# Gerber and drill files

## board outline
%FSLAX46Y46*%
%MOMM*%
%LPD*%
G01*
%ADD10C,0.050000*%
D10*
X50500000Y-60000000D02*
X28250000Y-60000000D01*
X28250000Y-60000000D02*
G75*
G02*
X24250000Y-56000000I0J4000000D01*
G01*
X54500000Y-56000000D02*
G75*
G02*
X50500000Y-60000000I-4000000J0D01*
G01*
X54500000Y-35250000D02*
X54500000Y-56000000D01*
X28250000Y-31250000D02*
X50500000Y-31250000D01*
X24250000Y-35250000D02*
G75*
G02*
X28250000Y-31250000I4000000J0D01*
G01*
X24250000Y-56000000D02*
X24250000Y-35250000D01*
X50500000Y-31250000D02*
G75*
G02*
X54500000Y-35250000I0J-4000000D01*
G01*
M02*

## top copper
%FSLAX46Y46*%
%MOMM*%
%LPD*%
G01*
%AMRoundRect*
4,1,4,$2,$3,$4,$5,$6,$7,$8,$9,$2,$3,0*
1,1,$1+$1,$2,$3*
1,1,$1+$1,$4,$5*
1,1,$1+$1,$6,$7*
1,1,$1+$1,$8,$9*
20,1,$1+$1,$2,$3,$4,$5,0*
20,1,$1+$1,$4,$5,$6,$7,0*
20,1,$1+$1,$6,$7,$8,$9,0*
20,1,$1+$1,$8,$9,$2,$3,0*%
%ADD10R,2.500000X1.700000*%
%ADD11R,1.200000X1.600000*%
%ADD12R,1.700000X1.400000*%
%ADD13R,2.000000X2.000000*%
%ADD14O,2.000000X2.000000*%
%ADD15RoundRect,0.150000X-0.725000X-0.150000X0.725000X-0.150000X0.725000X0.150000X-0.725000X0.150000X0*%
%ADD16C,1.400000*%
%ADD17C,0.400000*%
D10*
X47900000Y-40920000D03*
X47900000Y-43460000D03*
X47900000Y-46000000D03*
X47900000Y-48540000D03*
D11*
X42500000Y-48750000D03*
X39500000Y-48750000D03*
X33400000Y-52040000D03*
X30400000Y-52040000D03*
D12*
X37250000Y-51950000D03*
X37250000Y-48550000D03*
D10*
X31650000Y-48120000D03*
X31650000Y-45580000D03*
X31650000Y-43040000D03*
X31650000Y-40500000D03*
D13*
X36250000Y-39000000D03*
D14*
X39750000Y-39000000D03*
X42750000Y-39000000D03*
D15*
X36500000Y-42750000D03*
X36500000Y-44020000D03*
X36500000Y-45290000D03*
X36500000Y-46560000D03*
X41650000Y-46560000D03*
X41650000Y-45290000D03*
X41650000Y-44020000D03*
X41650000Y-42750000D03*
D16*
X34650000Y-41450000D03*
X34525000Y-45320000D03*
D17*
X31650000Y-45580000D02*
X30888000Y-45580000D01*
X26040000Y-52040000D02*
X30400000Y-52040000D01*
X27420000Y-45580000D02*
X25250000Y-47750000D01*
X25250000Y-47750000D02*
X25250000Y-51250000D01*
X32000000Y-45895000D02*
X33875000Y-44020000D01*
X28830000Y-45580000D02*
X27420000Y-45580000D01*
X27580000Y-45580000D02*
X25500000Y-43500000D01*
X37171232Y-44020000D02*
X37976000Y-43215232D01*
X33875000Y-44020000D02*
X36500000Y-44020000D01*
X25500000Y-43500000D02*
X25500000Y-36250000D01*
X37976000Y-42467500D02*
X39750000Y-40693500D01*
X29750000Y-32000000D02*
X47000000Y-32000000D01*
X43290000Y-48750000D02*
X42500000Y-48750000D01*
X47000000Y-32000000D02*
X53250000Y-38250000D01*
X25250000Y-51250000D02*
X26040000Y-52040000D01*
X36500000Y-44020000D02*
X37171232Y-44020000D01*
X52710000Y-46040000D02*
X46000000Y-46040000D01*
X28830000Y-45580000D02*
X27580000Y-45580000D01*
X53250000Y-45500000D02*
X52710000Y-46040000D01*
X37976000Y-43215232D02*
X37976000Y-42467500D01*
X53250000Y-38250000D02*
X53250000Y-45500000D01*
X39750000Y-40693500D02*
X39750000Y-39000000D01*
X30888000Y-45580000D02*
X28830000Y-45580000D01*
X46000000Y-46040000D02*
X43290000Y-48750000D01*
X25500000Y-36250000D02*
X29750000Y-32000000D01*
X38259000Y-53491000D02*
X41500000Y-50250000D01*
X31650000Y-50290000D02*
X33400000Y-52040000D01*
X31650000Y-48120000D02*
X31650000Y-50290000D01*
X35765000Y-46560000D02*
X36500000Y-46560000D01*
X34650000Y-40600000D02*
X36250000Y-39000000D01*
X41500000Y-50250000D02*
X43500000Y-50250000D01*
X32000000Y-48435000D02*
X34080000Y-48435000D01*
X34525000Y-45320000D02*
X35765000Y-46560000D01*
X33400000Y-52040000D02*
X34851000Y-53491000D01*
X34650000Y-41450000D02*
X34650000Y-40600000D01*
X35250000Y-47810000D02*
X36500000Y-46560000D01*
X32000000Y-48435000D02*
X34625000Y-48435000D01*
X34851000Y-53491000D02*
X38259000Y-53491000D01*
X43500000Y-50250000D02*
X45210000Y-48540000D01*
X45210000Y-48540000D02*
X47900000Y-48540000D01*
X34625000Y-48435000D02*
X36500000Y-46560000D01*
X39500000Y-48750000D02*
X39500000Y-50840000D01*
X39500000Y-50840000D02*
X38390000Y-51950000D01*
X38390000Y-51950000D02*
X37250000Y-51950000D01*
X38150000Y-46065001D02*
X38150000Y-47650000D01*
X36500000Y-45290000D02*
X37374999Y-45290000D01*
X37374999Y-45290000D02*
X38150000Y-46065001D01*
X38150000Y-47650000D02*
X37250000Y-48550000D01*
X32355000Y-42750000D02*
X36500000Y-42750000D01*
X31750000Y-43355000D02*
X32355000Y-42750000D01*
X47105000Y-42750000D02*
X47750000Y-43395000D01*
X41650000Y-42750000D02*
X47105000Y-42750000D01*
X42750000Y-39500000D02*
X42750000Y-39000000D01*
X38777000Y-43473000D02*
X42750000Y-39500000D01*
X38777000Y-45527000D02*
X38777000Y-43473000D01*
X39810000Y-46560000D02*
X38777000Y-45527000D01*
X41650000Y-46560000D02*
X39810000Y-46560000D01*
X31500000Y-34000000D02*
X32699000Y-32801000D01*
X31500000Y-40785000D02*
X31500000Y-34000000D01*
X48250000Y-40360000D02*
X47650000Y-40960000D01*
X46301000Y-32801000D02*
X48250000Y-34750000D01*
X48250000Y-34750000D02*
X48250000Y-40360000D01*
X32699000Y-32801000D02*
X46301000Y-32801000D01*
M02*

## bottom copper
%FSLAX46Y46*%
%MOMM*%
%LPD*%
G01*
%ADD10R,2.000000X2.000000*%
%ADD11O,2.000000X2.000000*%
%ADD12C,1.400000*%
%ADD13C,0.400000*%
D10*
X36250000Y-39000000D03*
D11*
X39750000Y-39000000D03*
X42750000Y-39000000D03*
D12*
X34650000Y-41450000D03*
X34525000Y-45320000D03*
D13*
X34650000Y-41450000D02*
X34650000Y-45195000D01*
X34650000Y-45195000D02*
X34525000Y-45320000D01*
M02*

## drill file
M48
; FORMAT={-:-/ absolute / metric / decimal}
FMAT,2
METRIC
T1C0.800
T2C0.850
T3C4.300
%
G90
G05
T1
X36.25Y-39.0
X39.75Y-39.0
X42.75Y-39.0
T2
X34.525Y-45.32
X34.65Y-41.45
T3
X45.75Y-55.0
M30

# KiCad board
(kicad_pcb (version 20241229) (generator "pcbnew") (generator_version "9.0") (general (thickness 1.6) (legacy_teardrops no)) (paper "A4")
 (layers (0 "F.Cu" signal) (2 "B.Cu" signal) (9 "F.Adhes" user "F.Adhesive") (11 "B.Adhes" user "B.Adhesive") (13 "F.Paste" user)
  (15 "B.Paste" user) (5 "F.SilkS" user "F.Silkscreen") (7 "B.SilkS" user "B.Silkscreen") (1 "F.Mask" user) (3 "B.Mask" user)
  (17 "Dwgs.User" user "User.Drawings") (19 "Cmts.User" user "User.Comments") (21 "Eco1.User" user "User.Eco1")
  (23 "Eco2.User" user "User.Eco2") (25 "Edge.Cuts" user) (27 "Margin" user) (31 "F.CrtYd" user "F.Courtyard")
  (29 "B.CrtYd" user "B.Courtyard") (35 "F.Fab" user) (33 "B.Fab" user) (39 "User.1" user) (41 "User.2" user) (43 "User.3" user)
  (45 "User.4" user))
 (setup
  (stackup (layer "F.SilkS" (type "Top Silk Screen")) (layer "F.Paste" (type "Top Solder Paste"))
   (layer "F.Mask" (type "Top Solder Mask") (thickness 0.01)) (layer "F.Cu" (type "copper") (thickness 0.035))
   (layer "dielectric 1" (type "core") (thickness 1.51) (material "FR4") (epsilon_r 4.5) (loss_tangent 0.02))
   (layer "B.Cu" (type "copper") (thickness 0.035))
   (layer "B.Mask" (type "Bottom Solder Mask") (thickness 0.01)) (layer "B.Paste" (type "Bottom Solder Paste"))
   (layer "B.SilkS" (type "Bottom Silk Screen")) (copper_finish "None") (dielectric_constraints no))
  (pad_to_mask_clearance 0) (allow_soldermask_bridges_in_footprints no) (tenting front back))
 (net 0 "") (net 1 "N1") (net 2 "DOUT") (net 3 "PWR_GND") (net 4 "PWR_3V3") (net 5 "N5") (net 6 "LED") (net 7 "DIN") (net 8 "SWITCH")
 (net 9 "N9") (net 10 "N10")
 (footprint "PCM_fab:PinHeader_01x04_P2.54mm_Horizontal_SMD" (layer "F.Cu") (at 47.9 40.92)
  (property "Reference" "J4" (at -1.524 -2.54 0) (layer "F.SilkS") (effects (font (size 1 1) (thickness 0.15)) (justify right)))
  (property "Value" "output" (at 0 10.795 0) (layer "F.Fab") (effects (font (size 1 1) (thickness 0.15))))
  (pad "1" smd rect (at 0 0) (size 2.5 1.7) (layers "F.Cu" "F.Mask" "F.Paste") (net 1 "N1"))
  (pad "2" smd rect (at 0 2.54) (size 2.5 1.7) (layers "F.Cu" "F.Mask" "F.Paste") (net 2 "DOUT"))
  (pad "3" smd rect (at 0 5.08) (size 2.5 1.7) (layers "F.Cu" "F.Mask" "F.Paste") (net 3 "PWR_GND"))
  (pad "4" smd rect (at 0 7.62) (size 2.5 1.7) (layers "F.Cu" "F.Mask" "F.Paste") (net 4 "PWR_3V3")))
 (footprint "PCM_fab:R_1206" (layer "F.Cu") (at 41 48.75 180)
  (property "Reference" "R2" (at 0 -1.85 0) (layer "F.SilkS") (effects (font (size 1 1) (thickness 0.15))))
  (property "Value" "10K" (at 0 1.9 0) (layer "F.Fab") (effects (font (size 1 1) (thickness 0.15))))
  (pad "1" smd rect (at -1.5 0 180) (size 1.2 1.6) (layers "F.Cu" "F.Mask" "F.Paste") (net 3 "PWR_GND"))
  (pad "2" smd rect (at 1.5 0 180) (size 1.2 1.6) (layers "F.Cu" "F.Mask" "F.Paste") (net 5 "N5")))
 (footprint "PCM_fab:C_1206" (layer "F.Cu") (at 31.9 52.04 180)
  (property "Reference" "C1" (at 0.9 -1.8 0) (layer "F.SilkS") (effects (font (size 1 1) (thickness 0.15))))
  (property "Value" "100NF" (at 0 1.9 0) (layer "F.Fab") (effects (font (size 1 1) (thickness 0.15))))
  (pad "1" smd rect (at -1.5 0 180) (size 1.2 1.6) (layers "F.Cu" "F.Mask" "F.Paste") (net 4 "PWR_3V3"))
  (pad "2" smd rect (at 1.5 0 180) (size 1.2 1.6) (layers "F.Cu" "F.Mask" "F.Paste") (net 3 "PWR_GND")))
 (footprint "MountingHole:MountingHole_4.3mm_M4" (layer "F.Cu") (at 45.75 55)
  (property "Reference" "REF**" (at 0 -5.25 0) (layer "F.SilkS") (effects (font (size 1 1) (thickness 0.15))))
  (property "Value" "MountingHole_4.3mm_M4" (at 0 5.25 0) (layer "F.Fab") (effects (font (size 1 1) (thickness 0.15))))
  (pad "" np_thru_hole circle (at 0 0) (size 4.3 4.3) (drill 4.3) (layers "*.Cu" "*.Mask")))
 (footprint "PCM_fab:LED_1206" (layer "F.Cu") (at 37.25 50.25 90)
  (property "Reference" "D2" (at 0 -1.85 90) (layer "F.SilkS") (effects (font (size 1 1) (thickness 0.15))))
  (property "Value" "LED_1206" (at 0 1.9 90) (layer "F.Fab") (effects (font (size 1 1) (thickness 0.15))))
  (pad "1" smd rect (at -1.7 0 90) (size 1.4 1.7) (layers "F.Cu" "F.Mask" "F.Paste") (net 5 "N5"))
  (pad "2" smd rect (at 1.7 0 90) (size 1.4 1.7) (layers "F.Cu" "F.Mask" "F.Paste") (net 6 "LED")))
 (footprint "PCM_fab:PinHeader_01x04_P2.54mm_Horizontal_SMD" (layer "F.Cu") (at 31.65 48.12 180)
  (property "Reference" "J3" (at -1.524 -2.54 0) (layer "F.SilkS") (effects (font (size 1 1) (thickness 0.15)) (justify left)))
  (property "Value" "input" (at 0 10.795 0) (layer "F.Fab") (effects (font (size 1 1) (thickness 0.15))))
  (pad "1" smd rect (at 0 0 180) (size 2.5 1.7) (layers "F.Cu" "F.Mask" "F.Paste") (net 4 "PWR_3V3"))
  (pad "2" smd rect (at 0 2.54 180) (size 2.5 1.7) (layers "F.Cu" "F.Mask" "F.Paste") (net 3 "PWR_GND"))
  (pad "3" smd rect (at 0 5.08 180) (size 2.5 1.7) (layers "F.Cu" "F.Mask" "F.Paste") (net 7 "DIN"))
  (pad "4" smd rect (at 0 7.62 180) (size 2.5 1.7) (layers "F.Cu" "F.Mask" "F.Paste") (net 1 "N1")))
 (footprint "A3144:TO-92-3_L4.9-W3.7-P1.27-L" (layer "F.Cu") (at 39.75 39)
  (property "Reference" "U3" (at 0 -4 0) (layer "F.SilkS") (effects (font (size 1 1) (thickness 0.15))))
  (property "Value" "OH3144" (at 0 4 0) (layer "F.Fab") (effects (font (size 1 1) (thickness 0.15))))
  (pad "1" thru_hole rect (at -3.5 0) (size 2 2) (drill 0.8) (layers "*.Cu" "*.Mask") (remove_unused_layers no) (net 4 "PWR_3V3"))
  (pad "2" thru_hole oval (at 0 0) (size 2 2) (drill 0.8) (layers "*.Cu" "*.Mask") (remove_unused_layers no) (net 3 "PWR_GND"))
  (pad "3" thru_hole oval (at 3 0) (size 2 2) (drill 0.8) (layers "*.Cu" "*.Mask") (remove_unused_layers no) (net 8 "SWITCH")))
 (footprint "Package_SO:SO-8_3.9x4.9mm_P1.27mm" (layer "F.Cu") (at 39.075 44.655)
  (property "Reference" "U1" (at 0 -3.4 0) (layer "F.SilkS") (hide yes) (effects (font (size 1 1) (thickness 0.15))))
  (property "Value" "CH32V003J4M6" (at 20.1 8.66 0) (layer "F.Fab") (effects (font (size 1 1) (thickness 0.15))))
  (pad "1" smd roundrect (at -2.575 -1.905) (size 1.75 0.6) (layers "F.Cu" "F.Mask" "F.Paste") (roundrect_rratio 0.25) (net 7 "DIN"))
  (pad "2" smd roundrect (at -2.575 -0.635) (size 1.75 0.6) (layers "F.Cu" "F.Mask" "F.Paste") (roundrect_rratio 0.25) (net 3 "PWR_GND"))
  (pad "3" smd roundrect (at -2.575 0.635) (size 1.75 0.6) (layers "F.Cu" "F.Mask" "F.Paste") (roundrect_rratio 0.25) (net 6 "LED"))
  (pad "4" smd roundrect (at -2.575 1.905) (size 1.75 0.6) (layers "F.Cu" "F.Mask" "F.Paste") (roundrect_rratio 0.25) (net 4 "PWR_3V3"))
  (pad "5" smd roundrect (at 2.575 1.905) (size 1.75 0.6) (layers "F.Cu" "F.Mask" "F.Paste") (roundrect_rratio 0.25) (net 8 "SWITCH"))
  (pad "6" smd roundrect (at 2.575 0.635) (size 1.75 0.6) (layers "F.Cu" "F.Mask" "F.Paste") (roundrect_rratio 0.25) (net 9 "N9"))
  (pad "7" smd roundrect (at 2.575 -0.635) (size 1.75 0.6) (layers "F.Cu" "F.Mask" "F.Paste") (roundrect_rratio 0.25) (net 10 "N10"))
  (pad "8" smd roundrect (at 2.575 -1.905) (size 1.75 0.6) (layers "F.Cu" "F.Mask" "F.Paste") (roundrect_rratio 0.25) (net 2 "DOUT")))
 (gr_line (start 50.5 60) (end 28.25 60) (stroke (width 0.05) (type default)) (layer "Edge.Cuts"))
 (gr_arc (start 28.25 60) (mid 25.421573 58.828427) (end 24.25 56) (stroke (width 0.05) (type default)) (layer "Edge.Cuts"))
 (gr_arc (start 54.5 56) (mid 53.328427 58.828427) (end 50.5 60) (stroke (width 0.05) (type default)) (layer "Edge.Cuts"))
 (gr_line (start 54.5 35.25) (end 54.5 56) (stroke (width 0.05) (type default)) (layer "Edge.Cuts"))
 (gr_line (start 28.25 31.25) (end 50.5 31.25) (stroke (width 0.05) (type default)) (layer "Edge.Cuts"))
 (gr_arc (start 24.25 35.25) (mid 25.421573 32.421573) (end 28.25 31.25) (stroke (width 0.05) (type default)) (layer "Edge.Cuts"))
 (gr_line (start 24.25 56) (end 24.25 35.25) (stroke (width 0.05) (type default)) (layer "Edge.Cuts"))
 (gr_arc (start 50.5 31.25) (mid 53.328427 32.421573) (end 54.5 35.25) (stroke (width 0.05) (type default)) (layer "Edge.Cuts"))
 (segment (start 31.65 45.58) (end 30.888 45.58) (width 0.4) (layer "F.Cu") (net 3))
 (segment (start 26.04 52.04) (end 30.4 52.04) (width 0.4) (layer "F.Cu") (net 3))
 (segment (start 27.42 45.58) (end 25.25 47.75) (width 0.4) (layer "F.Cu") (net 3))
 (segment (start 25.25 47.75) (end 25.25 51.25) (width 0.4) (layer "F.Cu") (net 3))
 (segment (start 32 45.895) (end 33.875 44.02) (width 0.4) (layer "F.Cu") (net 3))
 (segment (start 28.83 45.58) (end 27.42 45.58) (width 0.4) (layer "F.Cu") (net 3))
 (segment (start 27.58 45.58) (end 25.5 43.5) (width 0.4) (layer "F.Cu") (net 3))
 (segment (start 37.171232 44.02) (end 37.976 43.215232) (width 0.4) (layer "F.Cu") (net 3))
 (segment (start 33.875 44.02) (end 36.5 44.02) (width 0.4) (layer "F.Cu") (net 3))
 (segment (start 25.5 43.5) (end 25.5 36.25) (width 0.4) (layer "F.Cu") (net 3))
 (segment (start 37.976 42.4675) (end 39.75 40.6935) (width 0.4) (layer "F.Cu") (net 3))
 (segment (start 29.75 32) (end 47 32) (width 0.4) (layer "F.Cu") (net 3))
 (segment (start 43.29 48.75) (end 42.5 48.75) (width 0.4) (layer "F.Cu") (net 3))
 (segment (start 47 32) (end 53.25 38.25) (width 0.4) (layer "F.Cu") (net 3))
 (segment (start 25.25 51.25) (end 26.04 52.04) (width 0.4) (layer "F.Cu") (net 3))
 (segment (start 36.5 44.02) (end 37.171232 44.02) (width 0.4) (layer "F.Cu") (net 3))
 (segment (start 52.71 46.04) (end 46 46.04) (width 0.4) (layer "F.Cu") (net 3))
 (segment (start 28.83 45.58) (end 27.58 45.58) (width 0.4) (layer "F.Cu") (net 3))
 (segment (start 53.25 45.5) (end 52.71 46.04) (width 0.4) (layer "F.Cu") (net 3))
 (segment (start 37.976 43.215232) (end 37.976 42.4675) (width 0.4) (layer "F.Cu") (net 3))
 (segment (start 53.25 38.25) (end 53.25 45.5) (width 0.4) (layer "F.Cu") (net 3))
 (segment (start 39.75 40.6935) (end 39.75 39) (width 0.4) (layer "F.Cu") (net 3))
 (segment (start 30.888 45.58) (end 28.83 45.58) (width 0.4) (layer "F.Cu") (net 3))
 (segment (start 46 46.04) (end 43.29 48.75) (width 0.4) (layer "F.Cu") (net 3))
 (segment (start 25.5 36.25) (end 29.75 32) (width 0.4) (layer "F.Cu") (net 3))
 (segment (start 38.259 53.491) (end 41.5 50.25) (width 0.4) (layer "F.Cu") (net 4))
 (segment (start 31.65 50.29) (end 33.4 52.04) (width 0.4) (layer "F.Cu") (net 4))
 (segment (start 31.65 48.12) (end 31.65 50.29) (width 0.4) (layer "F.Cu") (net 4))
 (segment (start 35.765 46.56) (end 36.5 46.56) (width 0.4) (layer "F.Cu") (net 4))
 (segment (start 34.65 40.6) (end 36.25 39) (width 0.4) (layer "F.Cu") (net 4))
 (segment (start 41.5 50.25) (end 43.5 50.25) (width 0.4) (layer "F.Cu") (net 4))
 (segment (start 32 48.435) (end 34.08 48.435) (width 0.4) (layer "F.Cu") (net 4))
 (segment (start 34.525 45.32) (end 35.765 46.56) (width 0.4) (layer "F.Cu") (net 4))
 (segment (start 33.4 52.04) (end 34.851 53.491) (width 0.4) (layer "F.Cu") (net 4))
 (segment (start 34.65 41.45) (end 34.65 40.6) (width 0.4) (layer "F.Cu") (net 4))
 (segment (start 35.25 47.81) (end 36.5 46.56) (width 0.4) (layer "F.Cu") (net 4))
 (segment (start 32 48.435) (end 34.625 48.435) (width 0.4) (layer "F.Cu") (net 4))
 (segment (start 34.851 53.491) (end 38.259 53.491) (width 0.4) (layer "F.Cu") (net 4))
 (segment (start 43.5 50.25) (end 45.21 48.54) (width 0.4) (layer "F.Cu") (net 4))
 (segment (start 45.21 48.54) (end 47.9 48.54) (width 0.4) (layer "F.Cu") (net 4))
 (segment (start 34.625 48.435) (end 36.5 46.56) (width 0.4) (layer "F.Cu") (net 4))
 (via (at 34.65 41.45) (size 1.4) (drill 0.85) (layers "F.Cu" "B.Cu") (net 4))
 (via (at 34.525 45.32) (size 1.4) (drill 0.85) (layers "F.Cu" "B.Cu") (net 4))
 (segment (start 34.65 41.45) (end 34.65 45.195) (width 0.4) (layer "B.Cu") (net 4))
 (segment (start 34.65 45.195) (end 34.525 45.32) (width 0.4) (layer "B.Cu") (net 4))
 (segment (start 39.5 48.75) (end 39.5 50.84) (width 0.4) (layer "F.Cu") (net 5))
 (segment (start 39.5 50.84) (end 38.39 51.95) (width 0.4) (layer "F.Cu") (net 5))
 (segment (start 38.39 51.95) (end 37.25 51.95) (width 0.4) (layer "F.Cu") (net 5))
 (segment (start 38.15 46.065001) (end 38.15 47.65) (width 0.4) (layer "F.Cu") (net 6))
 (segment (start 36.5 45.29) (end 37.374999 45.29) (width 0.4) (layer "F.Cu") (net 6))
 (segment (start 37.374999 45.29) (end 38.15 46.065001) (width 0.4) (layer "F.Cu") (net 6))
 (segment (start 38.15 47.65) (end 37.25 48.55) (width 0.4) (layer "F.Cu") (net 6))
 (segment (start 32.355 42.75) (end 36.5 42.75) (width 0.4) (layer "F.Cu") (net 7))
 (segment (start 31.75 43.355) (end 32.355 42.75) (width 0.4) (layer "F.Cu") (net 7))
 (segment (start 47.105 42.75) (end 47.75 43.395) (width 0.4) (layer "F.Cu") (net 2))
 (segment (start 41.65 42.75) (end 47.105 42.75) (width 0.4) (layer "F.Cu") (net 2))
 (segment (start 42.75 39.5) (end 42.75 39) (width 0.4) (layer "F.Cu") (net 8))
 (segment (start 38.777 43.473) (end 42.75 39.5) (width 0.4) (layer "F.Cu") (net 8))
 (segment (start 38.777 45.527) (end 38.777 43.473) (width 0.4) (layer "F.Cu") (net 8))
 (segment (start 39.81 46.56) (end 38.777 45.527) (width 0.4) (layer "F.Cu") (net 8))
 (segment (start 41.65 46.56) (end 39.81 46.56) (width 0.4) (layer "F.Cu") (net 8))
 (segment (start 31.5 34) (end 32.699 32.801) (width 0.4) (layer "F.Cu") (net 1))
 (segment (start 31.5 40.785) (end 31.5 34) (width 0.4) (layer "F.Cu") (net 1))
 (segment (start 48.25 40.36) (end 47.65 40.96) (width 0.4) (layer "F.Cu") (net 1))
 (segment (start 46.301 32.801) (end 48.25 34.75) (width 0.4) (layer "F.Cu") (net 1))
 (segment (start 48.25 34.75) (end 48.25 40.36) (width 0.4) (layer "F.Cu") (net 1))
 (segment (start 32.699 32.801) (end 46.301 32.801) (width 0.4) (layer "F.Cu") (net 1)))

